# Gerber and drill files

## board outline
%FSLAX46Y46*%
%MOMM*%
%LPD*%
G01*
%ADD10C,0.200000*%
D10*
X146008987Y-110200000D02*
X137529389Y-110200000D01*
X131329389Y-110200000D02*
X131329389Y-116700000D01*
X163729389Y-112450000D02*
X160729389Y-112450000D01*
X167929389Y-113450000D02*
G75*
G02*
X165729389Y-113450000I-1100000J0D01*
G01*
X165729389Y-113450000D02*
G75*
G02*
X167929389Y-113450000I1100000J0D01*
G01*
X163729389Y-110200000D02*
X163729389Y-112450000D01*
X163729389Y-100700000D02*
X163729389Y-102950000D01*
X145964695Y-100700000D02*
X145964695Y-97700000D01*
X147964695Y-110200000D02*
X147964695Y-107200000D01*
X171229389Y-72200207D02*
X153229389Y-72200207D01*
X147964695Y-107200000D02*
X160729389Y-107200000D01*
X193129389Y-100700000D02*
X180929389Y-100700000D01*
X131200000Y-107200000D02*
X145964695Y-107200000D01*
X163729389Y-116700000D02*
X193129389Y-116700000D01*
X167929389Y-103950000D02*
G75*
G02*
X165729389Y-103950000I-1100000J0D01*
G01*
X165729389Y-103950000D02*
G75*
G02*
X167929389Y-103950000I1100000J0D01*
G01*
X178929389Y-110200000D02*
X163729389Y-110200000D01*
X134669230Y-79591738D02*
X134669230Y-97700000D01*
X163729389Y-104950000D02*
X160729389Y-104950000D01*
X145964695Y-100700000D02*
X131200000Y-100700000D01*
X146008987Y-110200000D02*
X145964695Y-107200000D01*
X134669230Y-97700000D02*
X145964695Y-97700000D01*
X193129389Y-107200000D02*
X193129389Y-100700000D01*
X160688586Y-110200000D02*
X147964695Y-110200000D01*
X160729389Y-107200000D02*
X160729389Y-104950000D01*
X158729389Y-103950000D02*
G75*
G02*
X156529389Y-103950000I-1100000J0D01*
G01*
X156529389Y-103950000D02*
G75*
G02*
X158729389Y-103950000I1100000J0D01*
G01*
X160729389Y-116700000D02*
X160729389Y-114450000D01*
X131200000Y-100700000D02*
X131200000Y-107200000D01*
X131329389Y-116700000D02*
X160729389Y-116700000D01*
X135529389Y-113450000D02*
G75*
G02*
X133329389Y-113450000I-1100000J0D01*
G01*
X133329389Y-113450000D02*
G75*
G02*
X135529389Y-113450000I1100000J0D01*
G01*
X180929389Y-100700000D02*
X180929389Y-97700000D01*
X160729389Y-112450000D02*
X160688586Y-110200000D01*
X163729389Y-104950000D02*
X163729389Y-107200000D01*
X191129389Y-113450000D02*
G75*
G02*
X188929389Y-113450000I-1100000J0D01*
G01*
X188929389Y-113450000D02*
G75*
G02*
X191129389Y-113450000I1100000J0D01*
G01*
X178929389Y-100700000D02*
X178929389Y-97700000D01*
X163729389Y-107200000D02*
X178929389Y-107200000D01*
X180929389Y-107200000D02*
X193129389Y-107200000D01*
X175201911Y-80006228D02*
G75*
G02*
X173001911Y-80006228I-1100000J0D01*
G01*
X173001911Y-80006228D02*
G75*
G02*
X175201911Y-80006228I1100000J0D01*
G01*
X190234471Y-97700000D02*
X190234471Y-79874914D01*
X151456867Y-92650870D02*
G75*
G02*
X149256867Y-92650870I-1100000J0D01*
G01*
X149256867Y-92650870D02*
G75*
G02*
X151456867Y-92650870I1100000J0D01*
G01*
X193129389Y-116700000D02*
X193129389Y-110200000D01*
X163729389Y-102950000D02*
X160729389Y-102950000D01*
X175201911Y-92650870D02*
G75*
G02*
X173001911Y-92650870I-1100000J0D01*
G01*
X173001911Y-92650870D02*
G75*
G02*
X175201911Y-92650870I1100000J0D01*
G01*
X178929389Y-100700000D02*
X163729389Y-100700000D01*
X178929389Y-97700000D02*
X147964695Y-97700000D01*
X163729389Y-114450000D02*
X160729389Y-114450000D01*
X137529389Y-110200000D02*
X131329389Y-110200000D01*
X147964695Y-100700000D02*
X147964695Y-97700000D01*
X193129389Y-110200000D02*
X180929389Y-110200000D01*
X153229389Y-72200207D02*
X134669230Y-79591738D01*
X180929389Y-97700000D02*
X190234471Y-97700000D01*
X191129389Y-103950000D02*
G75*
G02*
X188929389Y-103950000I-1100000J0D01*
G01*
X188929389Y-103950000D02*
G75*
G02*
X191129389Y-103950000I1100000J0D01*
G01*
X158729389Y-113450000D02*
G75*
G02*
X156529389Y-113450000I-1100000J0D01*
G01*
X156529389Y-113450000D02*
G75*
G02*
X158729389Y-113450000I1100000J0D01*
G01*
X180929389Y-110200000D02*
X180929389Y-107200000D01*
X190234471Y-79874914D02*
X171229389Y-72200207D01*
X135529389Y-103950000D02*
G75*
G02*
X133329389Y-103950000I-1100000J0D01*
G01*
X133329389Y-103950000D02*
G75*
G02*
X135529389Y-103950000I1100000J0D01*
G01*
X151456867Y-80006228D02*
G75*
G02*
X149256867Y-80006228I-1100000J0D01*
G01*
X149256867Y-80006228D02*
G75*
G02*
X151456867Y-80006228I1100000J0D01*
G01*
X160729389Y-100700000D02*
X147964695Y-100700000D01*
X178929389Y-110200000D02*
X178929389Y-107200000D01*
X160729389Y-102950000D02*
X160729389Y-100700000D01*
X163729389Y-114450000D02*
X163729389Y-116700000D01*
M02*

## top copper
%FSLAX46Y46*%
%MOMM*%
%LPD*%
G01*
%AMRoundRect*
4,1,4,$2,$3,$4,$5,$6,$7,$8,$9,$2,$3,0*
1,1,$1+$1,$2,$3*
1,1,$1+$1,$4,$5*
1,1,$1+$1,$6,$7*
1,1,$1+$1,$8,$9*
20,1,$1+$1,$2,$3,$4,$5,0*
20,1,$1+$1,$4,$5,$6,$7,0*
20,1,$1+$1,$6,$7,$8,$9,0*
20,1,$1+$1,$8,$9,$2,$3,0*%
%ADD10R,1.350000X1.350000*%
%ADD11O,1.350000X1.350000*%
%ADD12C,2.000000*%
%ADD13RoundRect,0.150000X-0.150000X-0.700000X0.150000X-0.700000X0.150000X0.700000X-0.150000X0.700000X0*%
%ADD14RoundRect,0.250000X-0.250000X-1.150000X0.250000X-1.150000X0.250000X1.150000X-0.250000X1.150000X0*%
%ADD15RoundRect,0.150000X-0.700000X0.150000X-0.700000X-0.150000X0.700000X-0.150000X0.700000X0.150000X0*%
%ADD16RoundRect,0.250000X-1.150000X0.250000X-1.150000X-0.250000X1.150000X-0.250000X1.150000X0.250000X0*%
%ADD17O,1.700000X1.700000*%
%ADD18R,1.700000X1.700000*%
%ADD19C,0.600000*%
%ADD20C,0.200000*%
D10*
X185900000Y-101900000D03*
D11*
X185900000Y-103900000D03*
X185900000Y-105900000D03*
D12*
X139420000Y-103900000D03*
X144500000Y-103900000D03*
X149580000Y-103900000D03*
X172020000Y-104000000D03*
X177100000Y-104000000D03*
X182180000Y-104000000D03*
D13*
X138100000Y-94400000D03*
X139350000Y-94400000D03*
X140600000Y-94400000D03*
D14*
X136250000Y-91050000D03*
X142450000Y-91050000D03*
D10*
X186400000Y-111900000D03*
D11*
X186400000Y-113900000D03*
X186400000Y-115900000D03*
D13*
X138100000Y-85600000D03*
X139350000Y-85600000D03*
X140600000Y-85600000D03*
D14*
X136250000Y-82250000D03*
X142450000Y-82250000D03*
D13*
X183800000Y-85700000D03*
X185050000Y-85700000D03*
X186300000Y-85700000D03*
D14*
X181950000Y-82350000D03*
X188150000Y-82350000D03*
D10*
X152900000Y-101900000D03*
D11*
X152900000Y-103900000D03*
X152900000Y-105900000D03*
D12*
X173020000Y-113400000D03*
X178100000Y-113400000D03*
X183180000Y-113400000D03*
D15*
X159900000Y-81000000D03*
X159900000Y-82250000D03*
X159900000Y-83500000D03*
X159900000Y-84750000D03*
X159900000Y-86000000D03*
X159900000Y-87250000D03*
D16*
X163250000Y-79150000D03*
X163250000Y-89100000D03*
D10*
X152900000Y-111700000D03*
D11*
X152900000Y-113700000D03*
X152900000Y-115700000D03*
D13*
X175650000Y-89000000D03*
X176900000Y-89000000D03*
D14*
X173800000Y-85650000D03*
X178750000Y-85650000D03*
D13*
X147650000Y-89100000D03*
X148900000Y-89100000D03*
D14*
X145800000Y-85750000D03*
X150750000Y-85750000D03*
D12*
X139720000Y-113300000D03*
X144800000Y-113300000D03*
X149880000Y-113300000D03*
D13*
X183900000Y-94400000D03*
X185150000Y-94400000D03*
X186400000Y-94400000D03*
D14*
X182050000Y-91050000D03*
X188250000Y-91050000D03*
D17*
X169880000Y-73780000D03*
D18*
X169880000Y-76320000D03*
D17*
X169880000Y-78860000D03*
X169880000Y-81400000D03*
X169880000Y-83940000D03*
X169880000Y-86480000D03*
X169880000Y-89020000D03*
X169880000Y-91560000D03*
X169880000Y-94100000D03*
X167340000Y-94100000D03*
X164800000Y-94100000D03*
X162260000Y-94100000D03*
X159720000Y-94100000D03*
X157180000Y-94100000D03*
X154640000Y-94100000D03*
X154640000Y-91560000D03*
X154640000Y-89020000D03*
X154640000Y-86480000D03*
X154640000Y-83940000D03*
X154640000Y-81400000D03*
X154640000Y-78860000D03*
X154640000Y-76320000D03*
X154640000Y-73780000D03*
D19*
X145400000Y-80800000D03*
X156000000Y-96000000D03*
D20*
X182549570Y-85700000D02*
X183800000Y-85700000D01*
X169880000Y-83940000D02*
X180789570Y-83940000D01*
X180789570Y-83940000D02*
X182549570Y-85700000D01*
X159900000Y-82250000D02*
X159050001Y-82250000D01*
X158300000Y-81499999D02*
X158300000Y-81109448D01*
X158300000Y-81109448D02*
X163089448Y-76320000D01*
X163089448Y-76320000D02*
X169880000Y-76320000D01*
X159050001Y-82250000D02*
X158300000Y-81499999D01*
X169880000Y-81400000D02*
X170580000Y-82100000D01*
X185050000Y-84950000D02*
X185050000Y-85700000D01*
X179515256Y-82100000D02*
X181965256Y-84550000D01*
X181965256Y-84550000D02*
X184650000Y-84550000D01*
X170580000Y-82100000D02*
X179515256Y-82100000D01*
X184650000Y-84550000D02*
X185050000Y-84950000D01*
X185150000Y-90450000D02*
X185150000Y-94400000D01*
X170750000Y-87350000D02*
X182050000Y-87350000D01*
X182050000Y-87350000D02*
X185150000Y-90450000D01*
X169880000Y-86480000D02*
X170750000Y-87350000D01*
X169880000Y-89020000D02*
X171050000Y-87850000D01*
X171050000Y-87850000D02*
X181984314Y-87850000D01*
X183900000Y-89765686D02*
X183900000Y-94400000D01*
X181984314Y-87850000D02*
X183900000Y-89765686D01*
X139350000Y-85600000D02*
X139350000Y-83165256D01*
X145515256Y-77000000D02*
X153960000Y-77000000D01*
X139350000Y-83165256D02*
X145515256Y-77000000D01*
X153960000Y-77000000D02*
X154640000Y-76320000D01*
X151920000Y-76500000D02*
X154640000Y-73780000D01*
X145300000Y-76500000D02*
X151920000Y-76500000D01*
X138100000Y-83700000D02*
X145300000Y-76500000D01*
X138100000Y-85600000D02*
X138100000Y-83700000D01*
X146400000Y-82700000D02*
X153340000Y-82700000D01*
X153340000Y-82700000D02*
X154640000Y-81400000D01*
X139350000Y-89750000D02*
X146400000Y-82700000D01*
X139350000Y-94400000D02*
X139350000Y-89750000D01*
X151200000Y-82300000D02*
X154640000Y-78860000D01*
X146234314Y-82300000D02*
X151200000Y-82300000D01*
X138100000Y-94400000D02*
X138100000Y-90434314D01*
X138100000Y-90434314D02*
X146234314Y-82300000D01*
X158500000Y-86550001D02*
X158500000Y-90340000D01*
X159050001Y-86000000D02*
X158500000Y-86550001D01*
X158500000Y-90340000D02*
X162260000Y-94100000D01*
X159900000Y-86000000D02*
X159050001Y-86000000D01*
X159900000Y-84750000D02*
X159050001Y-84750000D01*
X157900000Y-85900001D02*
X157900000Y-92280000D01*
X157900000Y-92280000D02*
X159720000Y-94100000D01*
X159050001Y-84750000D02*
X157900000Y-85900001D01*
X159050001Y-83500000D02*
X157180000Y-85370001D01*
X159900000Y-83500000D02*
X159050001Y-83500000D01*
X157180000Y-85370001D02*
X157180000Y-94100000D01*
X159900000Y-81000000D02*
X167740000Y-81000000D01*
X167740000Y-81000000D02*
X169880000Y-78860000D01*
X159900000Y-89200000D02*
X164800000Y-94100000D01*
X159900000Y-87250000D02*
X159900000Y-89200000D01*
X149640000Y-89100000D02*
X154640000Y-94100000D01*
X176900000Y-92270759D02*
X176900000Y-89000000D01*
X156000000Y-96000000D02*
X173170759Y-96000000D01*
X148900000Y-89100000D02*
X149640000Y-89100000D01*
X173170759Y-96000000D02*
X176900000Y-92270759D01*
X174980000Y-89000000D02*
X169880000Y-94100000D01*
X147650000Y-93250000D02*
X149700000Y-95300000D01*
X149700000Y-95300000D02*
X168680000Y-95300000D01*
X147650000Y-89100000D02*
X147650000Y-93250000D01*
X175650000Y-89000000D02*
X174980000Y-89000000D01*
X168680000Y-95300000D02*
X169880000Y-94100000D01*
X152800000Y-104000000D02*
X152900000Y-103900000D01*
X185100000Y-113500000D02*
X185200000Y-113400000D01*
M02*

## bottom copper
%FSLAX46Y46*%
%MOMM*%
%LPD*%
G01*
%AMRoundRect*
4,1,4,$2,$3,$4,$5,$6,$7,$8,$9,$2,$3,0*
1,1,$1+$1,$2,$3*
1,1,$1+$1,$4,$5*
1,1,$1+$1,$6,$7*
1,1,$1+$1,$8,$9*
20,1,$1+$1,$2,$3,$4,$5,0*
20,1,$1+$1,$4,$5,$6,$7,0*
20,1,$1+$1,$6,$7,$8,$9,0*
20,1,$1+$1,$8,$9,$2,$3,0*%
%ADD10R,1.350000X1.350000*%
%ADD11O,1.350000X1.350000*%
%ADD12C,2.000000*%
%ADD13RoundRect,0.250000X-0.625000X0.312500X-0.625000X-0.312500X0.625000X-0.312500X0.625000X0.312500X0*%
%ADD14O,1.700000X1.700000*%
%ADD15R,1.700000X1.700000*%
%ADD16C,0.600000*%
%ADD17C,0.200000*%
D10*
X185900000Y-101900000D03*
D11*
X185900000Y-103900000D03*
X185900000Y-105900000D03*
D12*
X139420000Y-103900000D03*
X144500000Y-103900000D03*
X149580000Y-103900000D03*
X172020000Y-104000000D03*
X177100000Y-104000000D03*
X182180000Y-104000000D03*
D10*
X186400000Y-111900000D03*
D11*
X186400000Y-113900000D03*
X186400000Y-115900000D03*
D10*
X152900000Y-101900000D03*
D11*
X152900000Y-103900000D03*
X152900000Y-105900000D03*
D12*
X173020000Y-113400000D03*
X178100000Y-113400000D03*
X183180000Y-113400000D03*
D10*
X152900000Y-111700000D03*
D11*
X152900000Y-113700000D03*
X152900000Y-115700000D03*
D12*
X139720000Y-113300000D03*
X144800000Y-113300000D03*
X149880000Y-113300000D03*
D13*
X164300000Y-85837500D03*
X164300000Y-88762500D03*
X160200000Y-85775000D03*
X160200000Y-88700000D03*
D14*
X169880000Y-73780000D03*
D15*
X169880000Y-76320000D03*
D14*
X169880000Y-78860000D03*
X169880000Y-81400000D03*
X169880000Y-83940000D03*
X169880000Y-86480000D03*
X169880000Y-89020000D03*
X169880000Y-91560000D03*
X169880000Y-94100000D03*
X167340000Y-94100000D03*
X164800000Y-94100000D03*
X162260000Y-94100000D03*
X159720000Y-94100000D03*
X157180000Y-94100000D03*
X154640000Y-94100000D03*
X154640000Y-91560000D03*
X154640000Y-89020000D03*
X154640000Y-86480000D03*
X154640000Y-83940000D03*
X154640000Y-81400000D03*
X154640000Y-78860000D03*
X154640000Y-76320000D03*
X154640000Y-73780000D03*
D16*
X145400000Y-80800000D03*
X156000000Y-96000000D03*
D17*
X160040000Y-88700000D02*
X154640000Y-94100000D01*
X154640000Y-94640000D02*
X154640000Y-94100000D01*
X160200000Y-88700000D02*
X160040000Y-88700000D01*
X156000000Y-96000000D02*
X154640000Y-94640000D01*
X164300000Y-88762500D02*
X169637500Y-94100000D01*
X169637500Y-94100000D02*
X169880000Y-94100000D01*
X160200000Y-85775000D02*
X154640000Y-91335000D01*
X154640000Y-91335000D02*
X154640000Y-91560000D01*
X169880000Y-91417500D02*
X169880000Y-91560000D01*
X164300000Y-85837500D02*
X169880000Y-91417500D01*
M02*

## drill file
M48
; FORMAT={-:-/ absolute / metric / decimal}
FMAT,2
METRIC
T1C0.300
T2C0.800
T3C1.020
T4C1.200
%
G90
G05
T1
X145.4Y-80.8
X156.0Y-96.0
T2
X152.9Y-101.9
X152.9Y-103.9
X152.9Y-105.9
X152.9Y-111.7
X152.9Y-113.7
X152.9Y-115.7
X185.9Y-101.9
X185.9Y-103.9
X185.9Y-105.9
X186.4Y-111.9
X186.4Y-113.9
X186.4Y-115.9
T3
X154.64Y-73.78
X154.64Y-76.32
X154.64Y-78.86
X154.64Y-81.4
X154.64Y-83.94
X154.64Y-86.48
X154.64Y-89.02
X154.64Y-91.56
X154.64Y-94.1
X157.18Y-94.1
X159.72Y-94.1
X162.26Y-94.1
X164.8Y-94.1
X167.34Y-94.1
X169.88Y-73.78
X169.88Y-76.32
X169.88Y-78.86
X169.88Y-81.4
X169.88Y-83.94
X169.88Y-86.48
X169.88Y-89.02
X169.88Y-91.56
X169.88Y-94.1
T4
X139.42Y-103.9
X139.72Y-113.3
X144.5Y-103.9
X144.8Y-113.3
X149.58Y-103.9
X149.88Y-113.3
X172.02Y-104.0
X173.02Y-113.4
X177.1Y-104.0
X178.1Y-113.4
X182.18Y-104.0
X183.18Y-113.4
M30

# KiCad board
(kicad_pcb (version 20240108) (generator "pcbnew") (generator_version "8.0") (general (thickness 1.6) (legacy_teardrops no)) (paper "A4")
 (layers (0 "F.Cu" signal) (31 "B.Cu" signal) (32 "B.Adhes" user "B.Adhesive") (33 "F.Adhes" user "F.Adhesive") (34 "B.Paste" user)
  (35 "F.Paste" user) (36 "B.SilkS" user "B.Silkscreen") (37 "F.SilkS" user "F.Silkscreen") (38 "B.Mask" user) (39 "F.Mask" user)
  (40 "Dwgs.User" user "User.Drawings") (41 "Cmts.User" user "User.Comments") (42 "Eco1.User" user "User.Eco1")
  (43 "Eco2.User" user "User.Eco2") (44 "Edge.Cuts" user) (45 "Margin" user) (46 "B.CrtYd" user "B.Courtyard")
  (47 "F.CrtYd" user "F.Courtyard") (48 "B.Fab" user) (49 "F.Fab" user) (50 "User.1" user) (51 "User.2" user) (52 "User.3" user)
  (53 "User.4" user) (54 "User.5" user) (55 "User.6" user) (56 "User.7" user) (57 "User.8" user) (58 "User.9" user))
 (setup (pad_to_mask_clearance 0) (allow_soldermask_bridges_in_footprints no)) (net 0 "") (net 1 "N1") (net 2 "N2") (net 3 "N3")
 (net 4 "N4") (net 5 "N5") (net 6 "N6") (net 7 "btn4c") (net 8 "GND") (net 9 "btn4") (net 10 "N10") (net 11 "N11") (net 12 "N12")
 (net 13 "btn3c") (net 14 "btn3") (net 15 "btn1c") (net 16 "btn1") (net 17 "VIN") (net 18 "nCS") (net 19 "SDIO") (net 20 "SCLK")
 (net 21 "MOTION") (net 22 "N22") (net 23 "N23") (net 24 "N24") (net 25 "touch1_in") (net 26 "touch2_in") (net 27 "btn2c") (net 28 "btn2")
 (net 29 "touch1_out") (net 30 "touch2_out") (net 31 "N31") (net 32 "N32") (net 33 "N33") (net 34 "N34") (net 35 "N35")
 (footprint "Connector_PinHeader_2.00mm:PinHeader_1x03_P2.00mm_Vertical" (layer "F.Cu") (at 185.9 101.9)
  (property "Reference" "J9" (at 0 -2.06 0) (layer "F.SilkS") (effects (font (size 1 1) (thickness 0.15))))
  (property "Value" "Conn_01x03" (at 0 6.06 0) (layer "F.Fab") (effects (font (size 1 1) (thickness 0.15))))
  (pad "1" thru_hole rect (at 0 0) (size 1.35 1.35) (drill 0.8) (layers "*.Cu" "*.Mask") (remove_unused_layers no) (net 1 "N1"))
  (pad "2" thru_hole oval (at 0 2) (size 1.35 1.35) (drill 0.8) (layers "*.Cu" "*.Mask") (remove_unused_layers no) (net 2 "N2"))
  (pad "3" thru_hole oval (at 0 4) (size 1.35 1.35) (drill 0.8) (layers "*.Cu" "*.Mask") (remove_unused_layers no) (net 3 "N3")))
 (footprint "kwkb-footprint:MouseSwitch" (layer "F.Cu") (at 144.5 103.9 90)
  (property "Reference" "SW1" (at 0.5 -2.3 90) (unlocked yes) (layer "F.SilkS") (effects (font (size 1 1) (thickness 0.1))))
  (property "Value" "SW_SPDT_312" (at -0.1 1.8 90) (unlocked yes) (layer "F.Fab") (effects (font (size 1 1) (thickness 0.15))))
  (pad "1" thru_hole circle (at 0 -5.08 90) (size 2 2) (drill 1.2) (layers "*.Cu" "*.Mask") (remove_unused_layers no) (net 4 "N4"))
  (pad "2" thru_hole circle (at 0 0 90) (size 2 2) (drill 1.2) (layers "*.Cu" "*.Mask") (remove_unused_layers no) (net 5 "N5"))
  (pad "3" thru_hole circle (at 0 5.08 90) (size 2 2) (drill 1.2) (layers "*.Cu" "*.Mask") (remove_unused_layers no) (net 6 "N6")))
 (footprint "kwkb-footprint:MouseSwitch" (layer "F.Cu") (at 177.1 104 90)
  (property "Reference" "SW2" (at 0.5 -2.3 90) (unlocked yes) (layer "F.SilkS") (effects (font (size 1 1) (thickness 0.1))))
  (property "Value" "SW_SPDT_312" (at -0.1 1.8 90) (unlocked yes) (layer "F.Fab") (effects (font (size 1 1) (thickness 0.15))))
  (pad "1" thru_hole circle (at 0 -5.08 90) (size 2 2) (drill 1.2) (layers "*.Cu" "*.Mask") (remove_unused_layers no) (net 1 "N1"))
  (pad "2" thru_hole circle (at 0 0 90) (size 2 2) (drill 1.2) (layers "*.Cu" "*.Mask") (remove_unused_layers no) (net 2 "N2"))
  (pad "3" thru_hole circle (at 0 5.08 90) (size 2 2) (drill 1.2) (layers "*.Cu" "*.Mask") (remove_unused_layers no) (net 3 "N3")))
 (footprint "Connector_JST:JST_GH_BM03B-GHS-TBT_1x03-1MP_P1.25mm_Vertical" (layer "F.Cu") (at 139.35 92.45)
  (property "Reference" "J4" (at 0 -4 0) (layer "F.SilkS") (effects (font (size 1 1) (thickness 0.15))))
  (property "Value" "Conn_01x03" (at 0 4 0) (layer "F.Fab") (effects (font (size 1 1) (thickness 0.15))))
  (pad "1" smd roundrect (at -1.25 1.95) (size 0.6 1.7) (layers "F.Cu" "F.Paste" "F.Mask") (roundrect_rratio 0.25) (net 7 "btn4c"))
  (pad "2" smd roundrect (at 0 1.95) (size 0.6 1.7) (layers "F.Cu" "F.Paste" "F.Mask") (roundrect_rratio 0.25) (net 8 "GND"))
  (pad "3" smd roundrect (at 1.25 1.95) (size 0.6 1.7) (layers "F.Cu" "F.Paste" "F.Mask") (roundrect_rratio 0.25) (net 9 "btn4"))
  (pad "MP" smd roundrect (at -3.1 -1.4) (size 1 2.8) (layers "F.Cu" "F.Paste" "F.Mask") (roundrect_rratio 0.25))
  (pad "MP" smd roundrect (at 3.1 -1.4) (size 1 2.8) (layers "F.Cu" "F.Paste" "F.Mask") (roundrect_rratio 0.25)))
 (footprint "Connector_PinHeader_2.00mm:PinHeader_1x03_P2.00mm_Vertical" (layer "F.Cu") (at 186.4 111.9)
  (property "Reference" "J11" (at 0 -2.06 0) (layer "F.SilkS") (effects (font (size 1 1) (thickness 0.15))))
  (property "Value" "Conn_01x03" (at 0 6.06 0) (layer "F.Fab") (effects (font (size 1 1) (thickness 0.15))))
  (pad "1" thru_hole rect (at 0 0) (size 1.35 1.35) (drill 0.8) (layers "*.Cu" "*.Mask") (remove_unused_layers no) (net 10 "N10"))
  (pad "2" thru_hole oval (at 0 2) (size 1.35 1.35) (drill 0.8) (layers "*.Cu" "*.Mask") (remove_unused_layers no) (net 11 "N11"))
  (pad "3" thru_hole oval (at 0 4) (size 1.35 1.35) (drill 0.8) (layers "*.Cu" "*.Mask") (remove_unused_layers no) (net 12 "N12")))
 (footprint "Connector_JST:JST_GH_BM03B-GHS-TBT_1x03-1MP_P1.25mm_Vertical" (layer "F.Cu") (at 139.35 83.65)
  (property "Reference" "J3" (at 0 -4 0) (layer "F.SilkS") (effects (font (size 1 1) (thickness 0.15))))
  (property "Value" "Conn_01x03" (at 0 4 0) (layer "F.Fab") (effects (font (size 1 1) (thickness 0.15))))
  (pad "1" smd roundrect (at -1.25 1.95) (size 0.6 1.7) (layers "F.Cu" "F.Paste" "F.Mask") (roundrect_rratio 0.25) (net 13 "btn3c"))
  (pad "2" smd roundrect (at 0 1.95) (size 0.6 1.7) (layers "F.Cu" "F.Paste" "F.Mask") (roundrect_rratio 0.25) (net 8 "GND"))
  (pad "3" smd roundrect (at 1.25 1.95) (size 0.6 1.7) (layers "F.Cu" "F.Paste" "F.Mask") (roundrect_rratio 0.25) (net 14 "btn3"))
  (pad "MP" smd roundrect (at -3.1 -1.4) (size 1 2.8) (layers "F.Cu" "F.Paste" "F.Mask") (roundrect_rratio 0.25))
  (pad "MP" smd roundrect (at 3.1 -1.4) (size 1 2.8) (layers "F.Cu" "F.Paste" "F.Mask") (roundrect_rratio 0.25)))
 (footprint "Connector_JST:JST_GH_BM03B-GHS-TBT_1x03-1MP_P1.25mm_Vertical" (layer "F.Cu") (at 185.05 83.75)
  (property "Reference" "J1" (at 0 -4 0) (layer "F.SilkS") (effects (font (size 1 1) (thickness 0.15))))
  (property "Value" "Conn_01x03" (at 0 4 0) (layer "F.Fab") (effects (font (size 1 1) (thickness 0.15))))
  (pad "1" smd roundrect (at -1.25 1.95) (size 0.6 1.7) (layers "F.Cu" "F.Paste" "F.Mask") (roundrect_rratio 0.25) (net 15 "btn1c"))
  (pad "2" smd roundrect (at 0 1.95) (size 0.6 1.7) (layers "F.Cu" "F.Paste" "F.Mask") (roundrect_rratio 0.25) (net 8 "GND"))
  (pad "3" smd roundrect (at 1.25 1.95) (size 0.6 1.7) (layers "F.Cu" "F.Paste" "F.Mask") (roundrect_rratio 0.25) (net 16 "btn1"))
  (pad "MP" smd roundrect (at -3.1 -1.4) (size 1 2.8) (layers "F.Cu" "F.Paste" "F.Mask") (roundrect_rratio 0.25))
  (pad "MP" smd roundrect (at 3.1 -1.4) (size 1 2.8) (layers "F.Cu" "F.Paste" "F.Mask") (roundrect_rratio 0.25)))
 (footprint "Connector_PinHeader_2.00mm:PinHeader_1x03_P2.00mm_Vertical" (layer "F.Cu") (at 152.9 101.9)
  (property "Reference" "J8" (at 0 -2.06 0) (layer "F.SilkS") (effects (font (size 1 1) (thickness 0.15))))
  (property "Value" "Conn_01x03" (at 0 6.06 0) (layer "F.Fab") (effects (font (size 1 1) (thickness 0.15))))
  (pad "1" thru_hole rect (at 0 0) (size 1.35 1.35) (drill 0.8) (layers "*.Cu" "*.Mask") (remove_unused_layers no) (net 4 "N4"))
  (pad "2" thru_hole oval (at 0 2) (size 1.35 1.35) (drill 0.8) (layers "*.Cu" "*.Mask") (remove_unused_layers no) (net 5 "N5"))
  (pad "3" thru_hole oval (at 0 4) (size 1.35 1.35) (drill 0.8) (layers "*.Cu" "*.Mask") (remove_unused_layers no) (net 6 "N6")))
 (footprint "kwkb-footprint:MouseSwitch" (layer "F.Cu") (at 178.1 113.4 90)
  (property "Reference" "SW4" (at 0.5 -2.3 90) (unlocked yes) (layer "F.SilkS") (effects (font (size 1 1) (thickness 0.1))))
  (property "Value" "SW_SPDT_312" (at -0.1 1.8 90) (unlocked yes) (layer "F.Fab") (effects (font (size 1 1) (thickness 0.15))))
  (pad "1" thru_hole circle (at 0 -5.08 90) (size 2 2) (drill 1.2) (layers "*.Cu" "*.Mask") (remove_unused_layers no) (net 10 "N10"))
  (pad "2" thru_hole circle (at 0 0 90) (size 2 2) (drill 1.2) (layers "*.Cu" "*.Mask") (remove_unused_layers no) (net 11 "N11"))
  (pad "3" thru_hole circle (at 0 5.08 90) (size 2 2) (drill 1.2) (layers "*.Cu" "*.Mask") (remove_unused_layers no) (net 12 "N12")))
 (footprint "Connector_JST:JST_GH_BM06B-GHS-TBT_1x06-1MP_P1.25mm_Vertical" (layer "F.Cu") (at 161.85 84.125 -90)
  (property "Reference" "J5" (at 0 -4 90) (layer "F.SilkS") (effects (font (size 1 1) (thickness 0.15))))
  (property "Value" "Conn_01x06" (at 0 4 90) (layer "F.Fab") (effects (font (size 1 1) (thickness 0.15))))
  (pad "1" smd roundrect (at -3.125 1.95 270) (size 0.6 1.7) (layers "F.Cu" "F.Paste" "F.Mask") (roundrect_rratio 0.25) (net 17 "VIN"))
  (pad "2" smd roundrect (at -1.875 1.95 270) (size 0.6 1.7) (layers "F.Cu" "F.Paste" "F.Mask") (roundrect_rratio 0.25) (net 8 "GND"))
  (pad "3" smd roundrect (at -0.625 1.95 270) (size 0.6 1.7) (layers "F.Cu" "F.Paste" "F.Mask") (roundrect_rratio 0.25) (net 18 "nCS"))
  (pad "4" smd roundrect (at 0.625 1.95 270) (size 0.6 1.7) (layers "F.Cu" "F.Paste" "F.Mask") (roundrect_rratio 0.25) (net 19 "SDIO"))
  (pad "5" smd roundrect (at 1.875 1.95 270) (size 0.6 1.7) (layers "F.Cu" "F.Paste" "F.Mask") (roundrect_rratio 0.25) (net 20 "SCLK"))
  (pad "6" smd roundrect (at 3.125 1.95 270) (size 0.6 1.7) (layers "F.Cu" "F.Paste" "F.Mask") (roundrect_rratio 0.25) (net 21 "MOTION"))
  (pad "MP" smd roundrect (at -4.975 -1.4 270) (size 1 2.8) (layers "F.Cu" "F.Paste" "F.Mask") (roundrect_rratio 0.25))
  (pad "MP" smd roundrect (at 4.975 -1.4 270) (size 1 2.8) (layers "F.Cu" "F.Paste" "F.Mask") (roundrect_rratio 0.25)))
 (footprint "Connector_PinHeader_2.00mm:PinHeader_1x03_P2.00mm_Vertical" (layer "F.Cu") (at 152.9 111.7)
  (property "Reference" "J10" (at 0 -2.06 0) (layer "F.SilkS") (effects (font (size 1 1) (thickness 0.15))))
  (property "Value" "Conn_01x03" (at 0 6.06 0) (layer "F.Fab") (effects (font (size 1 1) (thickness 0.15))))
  (pad "1" thru_hole rect (at 0 0) (size 1.35 1.35) (drill 0.8) (layers "*.Cu" "*.Mask") (remove_unused_layers no) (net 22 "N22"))
  (pad "2" thru_hole oval (at 0 2) (size 1.35 1.35) (drill 0.8) (layers "*.Cu" "*.Mask") (remove_unused_layers no) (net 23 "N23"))
  (pad "3" thru_hole oval (at 0 4) (size 1.35 1.35) (drill 0.8) (layers "*.Cu" "*.Mask") (remove_unused_layers no) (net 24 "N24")))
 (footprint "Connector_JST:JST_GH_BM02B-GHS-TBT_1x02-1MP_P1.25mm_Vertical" (layer "F.Cu") (at 176.275 87.05)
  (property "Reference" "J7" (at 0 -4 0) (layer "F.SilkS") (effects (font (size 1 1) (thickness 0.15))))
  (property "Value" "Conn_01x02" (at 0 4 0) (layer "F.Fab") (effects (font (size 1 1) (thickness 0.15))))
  (pad "1" smd roundrect (at -0.625 1.95) (size 0.6 1.7) (layers "F.Cu" "F.Paste" "F.Mask") (roundrect_rratio 0.25) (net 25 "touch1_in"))
  (pad "2" smd roundrect (at 0.625 1.95) (size 0.6 1.7) (layers "F.Cu" "F.Paste" "F.Mask") (roundrect_rratio 0.25) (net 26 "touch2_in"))
  (pad "MP" smd roundrect (at -2.475 -1.4) (size 1 2.8) (layers "F.Cu" "F.Paste" "F.Mask") (roundrect_rratio 0.25))
  (pad "MP" smd roundrect (at 2.475 -1.4) (size 1 2.8) (layers "F.Cu" "F.Paste" "F.Mask") (roundrect_rratio 0.25)))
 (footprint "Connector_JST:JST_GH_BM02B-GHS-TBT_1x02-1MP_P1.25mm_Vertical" (layer "F.Cu") (at 148.275 87.15)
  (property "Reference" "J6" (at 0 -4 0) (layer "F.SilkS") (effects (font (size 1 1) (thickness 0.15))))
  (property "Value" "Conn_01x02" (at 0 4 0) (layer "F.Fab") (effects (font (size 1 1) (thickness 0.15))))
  (pad "1" smd roundrect (at -0.625 1.95) (size 0.6 1.7) (layers "F.Cu" "F.Paste" "F.Mask") (roundrect_rratio 0.25) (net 25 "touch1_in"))
  (pad "2" smd roundrect (at 0.625 1.95) (size 0.6 1.7) (layers "F.Cu" "F.Paste" "F.Mask") (roundrect_rratio 0.25) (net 26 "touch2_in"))
  (pad "MP" smd roundrect (at -2.475 -1.4) (size 1 2.8) (layers "F.Cu" "F.Paste" "F.Mask") (roundrect_rratio 0.25))
  (pad "MP" smd roundrect (at 2.475 -1.4) (size 1 2.8) (layers "F.Cu" "F.Paste" "F.Mask") (roundrect_rratio 0.25)))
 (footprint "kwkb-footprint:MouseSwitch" (layer "F.Cu") (at 144.8 113.3 90)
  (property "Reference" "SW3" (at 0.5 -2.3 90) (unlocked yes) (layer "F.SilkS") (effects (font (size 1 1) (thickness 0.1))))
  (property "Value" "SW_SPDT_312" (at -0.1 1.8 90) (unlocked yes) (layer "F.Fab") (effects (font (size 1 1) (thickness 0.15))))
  (pad "1" thru_hole circle (at 0 -5.08 90) (size 2 2) (drill 1.2) (layers "*.Cu" "*.Mask") (remove_unused_layers no) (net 22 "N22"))
  (pad "2" thru_hole circle (at 0 0 90) (size 2 2) (drill 1.2) (layers "*.Cu" "*.Mask") (remove_unused_layers no) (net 23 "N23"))
  (pad "3" thru_hole circle (at 0 5.08 90) (size 2 2) (drill 1.2) (layers "*.Cu" "*.Mask") (remove_unused_layers no) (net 24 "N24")))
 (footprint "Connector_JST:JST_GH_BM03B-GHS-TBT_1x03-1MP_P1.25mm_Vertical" (layer "F.Cu") (at 185.15 92.45)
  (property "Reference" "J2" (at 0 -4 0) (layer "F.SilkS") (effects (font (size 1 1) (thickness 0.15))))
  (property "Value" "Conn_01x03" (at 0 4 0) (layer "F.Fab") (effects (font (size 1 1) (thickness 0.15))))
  (pad "1" smd roundrect (at -1.25 1.95) (size 0.6 1.7) (layers "F.Cu" "F.Paste" "F.Mask") (roundrect_rratio 0.25) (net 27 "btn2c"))
  (pad "2" smd roundrect (at 0 1.95) (size 0.6 1.7) (layers "F.Cu" "F.Paste" "F.Mask") (roundrect_rratio 0.25) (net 8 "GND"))
  (pad "3" smd roundrect (at 1.25 1.95) (size 0.6 1.7) (layers "F.Cu" "F.Paste" "F.Mask") (roundrect_rratio 0.25) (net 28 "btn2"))
  (pad "MP" smd roundrect (at -3.1 -1.4) (size 1 2.8) (layers "F.Cu" "F.Paste" "F.Mask") (roundrect_rratio 0.25))
  (pad "MP" smd roundrect (at 3.1 -1.4) (size 1 2.8) (layers "F.Cu" "F.Paste" "F.Mask") (roundrect_rratio 0.25)))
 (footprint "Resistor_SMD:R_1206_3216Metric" (layer "B.Cu") (at 164.3 87.3 -90)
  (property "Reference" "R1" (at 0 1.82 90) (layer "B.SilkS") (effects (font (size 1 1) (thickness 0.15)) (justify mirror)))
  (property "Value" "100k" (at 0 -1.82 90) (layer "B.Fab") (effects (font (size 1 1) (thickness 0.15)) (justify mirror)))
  (pad "1" smd roundrect (at -1.4625 0 270) (size 1.125 1.75) (layers "B.Cu" "B.Paste" "B.Mask") (roundrect_rratio 0.222222)
   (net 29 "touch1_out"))
  (pad "2" smd roundrect (at 1.4625 0 270) (size 1.125 1.75) (layers "B.Cu" "B.Paste" "B.Mask") (roundrect_rratio 0.222222)
   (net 25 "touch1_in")))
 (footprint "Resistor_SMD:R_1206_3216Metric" (layer "B.Cu") (at 160.2 87.2375 -90)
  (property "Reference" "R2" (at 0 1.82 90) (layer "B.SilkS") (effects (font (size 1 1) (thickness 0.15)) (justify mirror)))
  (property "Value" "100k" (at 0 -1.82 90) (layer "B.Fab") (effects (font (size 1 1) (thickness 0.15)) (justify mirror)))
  (pad "1" smd roundrect (at -1.4625 0 270) (size 1.125 1.75) (layers "B.Cu" "B.Paste" "B.Mask") (roundrect_rratio 0.222222)
   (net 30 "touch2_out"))
  (pad "2" smd roundrect (at 1.4625 0 270) (size 1.125 1.75) (layers "B.Cu" "B.Paste" "B.Mask") (roundrect_rratio 0.222222)
   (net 26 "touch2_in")))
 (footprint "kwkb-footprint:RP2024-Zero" (layer "B.Cu") (at 162.26 72.19 180)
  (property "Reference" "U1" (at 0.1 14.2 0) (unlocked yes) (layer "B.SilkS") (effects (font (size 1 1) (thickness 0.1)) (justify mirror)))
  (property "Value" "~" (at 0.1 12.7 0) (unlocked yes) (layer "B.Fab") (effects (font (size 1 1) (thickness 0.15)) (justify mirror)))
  (pad "1" thru_hole oval (at -7.62 -1.59 180) (size 1.7 1.7) (drill 1.02) (layers "*.Cu" "*.Mask") (remove_unused_layers no) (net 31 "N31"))
  (pad "2" thru_hole rect (at -7.62 -4.13 180) (size 1.7 1.7) (drill 1.02) (layers "*.Cu" "*.Mask") (remove_unused_layers no) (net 8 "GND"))
  (pad "3" thru_hole oval (at -7.62 -6.67 180) (size 1.7 1.7) (drill 1.02) (layers "*.Cu" "*.Mask") (remove_unused_layers no) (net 17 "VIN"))
  (pad "4" thru_hole oval (at -7.62 -9.21 180) (size 1.7 1.7) (drill 1.02) (layers "*.Cu" "*.Mask") (remove_unused_layers no)
   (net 16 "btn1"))
  (pad "5" thru_hole oval (at -7.62 -11.75 180) (size 1.7 1.7) (drill 1.02) (layers "*.Cu" "*.Mask") (remove_unused_layers no)
   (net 15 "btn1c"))
  (pad "6" thru_hole oval (at -7.62 -14.29 180) (size 1.7 1.7) (drill 1.02) (layers "*.Cu" "*.Mask") (remove_unused_layers no)
   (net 28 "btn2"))
  (pad "7" thru_hole oval (at -7.62 -16.83 180) (size 1.7 1.7) (drill 1.02) (layers "*.Cu" "*.Mask") (remove_unused_layers no)
   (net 27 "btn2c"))
  (pad "8" thru_hole oval (at -7.62 -19.37 180) (size 1.7 1.7) (drill 1.02) (layers "*.Cu" "*.Mask") (remove_unused_layers no)
   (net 29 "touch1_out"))
  (pad "9" thru_hole oval (at -7.62 -21.91 180) (size 1.7 1.7) (drill 1.02) (layers "*.Cu" "*.Mask") (remove_unused_layers no)
   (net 25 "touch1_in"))
  (pad "10" thru_hole oval (at -5.08 -21.91 180) (size 1.7 1.7) (drill 1.02) (layers "*.Cu" "*.Mask") (remove_unused_layers no)
   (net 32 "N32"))
  (pad "11" thru_hole oval (at -2.54 -21.91 180) (size 1.7 1.7) (drill 1.02) (layers "*.Cu" "*.Mask") (remove_unused_layers no)
   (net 21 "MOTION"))
  (pad "12" thru_hole oval (at 0 -21.91 180) (size 1.7 1.7) (drill 1.02) (layers "*.Cu" "*.Mask") (remove_unused_layers no) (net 20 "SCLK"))
  (pad "13" thru_hole oval (at 2.54 -21.91 180) (size 1.7 1.7) (drill 1.02) (layers "*.Cu" "*.Mask") (remove_unused_layers no)
   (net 19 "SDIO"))
  (pad "14" thru_hole oval (at 5.08 -21.91 180) (size 1.7 1.7) (drill 1.02) (layers "*.Cu" "*.Mask") (remove_unused_layers no)
   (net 18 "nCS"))
  (pad "15" thru_hole oval (at 7.62 -21.91 180) (size 1.7 1.7) (drill 1.02) (layers "*.Cu" "*.Mask") (remove_unused_layers no)
   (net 26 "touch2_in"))
  (pad "16" thru_hole oval (at 7.62 -19.37 180) (size 1.7 1.7) (drill 1.02) (layers "*.Cu" "*.Mask") (remove_unused_layers no)
   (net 30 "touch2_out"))
  (pad "17" thru_hole oval (at 7.62 -16.83 180) (size 1.7 1.7) (drill 1.02) (layers "*.Cu" "*.Mask") (remove_unused_layers no)
   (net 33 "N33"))
  (pad "18" thru_hole oval (at 7.62 -14.29 180) (size 1.7 1.7) (drill 1.02) (layers "*.Cu" "*.Mask") (remove_unused_layers no)
   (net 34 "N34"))
  (pad "19" thru_hole oval (at 7.62 -11.75 180) (size 1.7 1.7) (drill 1.02) (layers "*.Cu" "*.Mask") (remove_unused_layers no)
   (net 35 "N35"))
  (pad "20" thru_hole oval (at 7.62 -9.21 180) (size 1.7 1.7) (drill 1.02) (layers "*.Cu" "*.Mask") (remove_unused_layers no) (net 9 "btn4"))
  (pad "21" thru_hole oval (at 7.62 -6.67 180) (size 1.7 1.7) (drill 1.02) (layers "*.Cu" "*.Mask") (remove_unused_layers no)
   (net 7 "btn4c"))
  (pad "22" thru_hole oval (at 7.62 -4.13 180) (size 1.7 1.7) (drill 1.02) (layers "*.Cu" "*.Mask") (remove_unused_layers no)
   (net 14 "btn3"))
  (pad "23" thru_hole oval (at 7.62 -1.59 180) (size 1.7 1.7) (drill 1.02) (layers "*.Cu" "*.Mask") (remove_unused_layers no)
   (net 13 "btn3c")))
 (gr_line (start 146.008987 110.2) (end 137.529389 110.2) (stroke (width 0.2) (type default)) (layer "Edge.Cuts"))
 (gr_line (start 131.329389 110.2) (end 131.329389 116.7) (stroke (width 0.2) (type default)) (layer "Edge.Cuts"))
 (gr_line (start 163.729389 112.45) (end 160.729389 112.45) (stroke (width 0.2) (type default)) (layer "Edge.Cuts"))
 (gr_circle (center 166.829389 113.45) (end 165.729389 113.45) (stroke (width 0.2) (type default)) (fill none) (layer "Edge.Cuts"))
 (gr_line (start 163.729389 110.2) (end 163.729389 112.45) (stroke (width 0.2) (type default)) (layer "Edge.Cuts"))
 (gr_line (start 163.729389 100.7) (end 163.729389 102.95) (stroke (width 0.2) (type default)) (layer "Edge.Cuts"))
 (gr_line (start 145.964695 100.7) (end 145.964695 97.7) (stroke (width 0.2) (type default)) (layer "Edge.Cuts"))
 (gr_line (start 147.964695 110.2) (end 147.964695 107.2) (stroke (width 0.2) (type default)) (layer "Edge.Cuts"))
 (gr_line (start 171.229389 72.200207) (end 153.229389 72.200207) (stroke (width 0.2) (type default)) (layer "Edge.Cuts"))
 (gr_line (start 147.964695 107.2) (end 160.729389 107.2) (stroke (width 0.2) (type default)) (layer "Edge.Cuts"))
 (gr_line (start 193.129389 100.7) (end 180.929389 100.7) (stroke (width 0.2) (type default)) (layer "Edge.Cuts"))
 (gr_line (start 131.2 107.2) (end 145.964695 107.2) (stroke (width 0.2) (type default)) (layer "Edge.Cuts"))
 (gr_line (start 163.729389 116.7) (end 193.129389 116.7) (stroke (width 0.2) (type default)) (layer "Edge.Cuts"))
 (gr_circle (center 166.829389 103.95) (end 165.729389 103.95) (stroke (width 0.2) (type default)) (fill none) (layer "Edge.Cuts"))
 (gr_line (start 178.929389 110.2) (end 163.729389 110.2) (stroke (width 0.2) (type default)) (layer "Edge.Cuts"))
 (gr_line (start 134.66923 79.591738) (end 134.66923 97.7) (stroke (width 0.2) (type default)) (layer "Edge.Cuts"))
 (gr_line (start 163.729389 104.95) (end 160.729389 104.95) (stroke (width 0.2) (type default)) (layer "Edge.Cuts"))
 (gr_line (start 145.964695 100.7) (end 131.2 100.7) (stroke (width 0.2) (type default)) (layer "Edge.Cuts"))
 (gr_line (start 146.008987 110.2) (end 145.964695 107.2) (stroke (width 0.2) (type default)) (layer "Edge.Cuts"))
 (gr_line (start 134.66923 97.7) (end 145.964695 97.7) (stroke (width 0.2) (type default)) (layer "Edge.Cuts"))
 (gr_line (start 193.129389 107.2) (end 193.129389 100.7) (stroke (width 0.2) (type default)) (layer "Edge.Cuts"))
 (gr_line (start 160.688586 110.2) (end 147.964695 110.2) (stroke (width 0.2) (type default)) (layer "Edge.Cuts"))
 (gr_line (start 160.729389 107.2) (end 160.729389 104.95) (stroke (width 0.2) (type default)) (layer "Edge.Cuts"))
 (gr_circle (center 157.629389 103.95) (end 156.529389 103.95) (stroke (width 0.2) (type default)) (fill none) (layer "Edge.Cuts"))
 (gr_line (start 160.729389 116.7) (end 160.729389 114.45) (stroke (width 0.2) (type default)) (layer "Edge.Cuts"))
 (gr_line (start 131.2 100.7) (end 131.2 107.2) (stroke (width 0.2) (type default)) (layer "Edge.Cuts"))
 (gr_line (start 131.329389 116.7) (end 160.729389 116.7) (stroke (width 0.2) (type default)) (layer "Edge.Cuts"))
 (gr_circle (center 134.429389 113.45) (end 133.329389 113.45) (stroke (width 0.2) (type default)) (fill none) (layer "Edge.Cuts"))
 (gr_line (start 180.929389 100.7) (end 180.929389 97.7) (stroke (width 0.2) (type default)) (layer "Edge.Cuts"))
 (gr_line (start 160.729389 112.45) (end 160.688586 110.2) (stroke (width 0.2) (type default)) (layer "Edge.Cuts"))
 (gr_line (start 163.729389 104.95) (end 163.729389 107.2) (stroke (width 0.2) (type default)) (layer "Edge.Cuts"))
 (gr_circle (center 190.029389 113.45) (end 188.929389 113.45) (stroke (width 0.2) (type default)) (fill none) (layer "Edge.Cuts"))
 (gr_line (start 178.929389 100.7) (end 178.929389 97.7) (stroke (width 0.2) (type default)) (layer "Edge.Cuts"))
 (gr_line (start 163.729389 107.2) (end 178.929389 107.2) (stroke (width 0.2) (type default)) (layer "Edge.Cuts"))
 (gr_line (start 180.929389 107.2) (end 193.129389 107.2) (stroke (width 0.2) (type default)) (layer "Edge.Cuts"))
 (gr_circle (center 174.101911 80.006228) (end 173.001911 80.006228) (stroke (width 0.2) (type default)) (fill none) (layer "Edge.Cuts"))
 (gr_line (start 190.234471 97.7) (end 190.234471 79.874914) (stroke (width 0.2) (type default)) (layer "Edge.Cuts"))
 (gr_circle (center 150.356867 92.65087) (end 149.256867 92.65087) (stroke (width 0.2) (type default)) (fill none) (layer "Edge.Cuts"))
 (gr_line (start 193.129389 116.7) (end 193.129389 110.2) (stroke (width 0.2) (type default)) (layer "Edge.Cuts"))
 (gr_line (start 163.729389 102.95) (end 160.729389 102.95) (stroke (width 0.2) (type default)) (layer "Edge.Cuts"))
 (gr_circle (center 174.101911 92.65087) (end 173.001911 92.65087) (stroke (width 0.2) (type default)) (fill none) (layer "Edge.Cuts"))
 (gr_line (start 178.929389 100.7) (end 163.729389 100.7) (stroke (width 0.2) (type default)) (layer "Edge.Cuts"))
 (gr_line (start 178.929389 97.7) (end 147.964695 97.7) (stroke (width 0.2) (type default)) (layer "Edge.Cuts"))
 (gr_line (start 163.729389 114.45) (end 160.729389 114.45) (stroke (width 0.2) (type default)) (layer "Edge.Cuts"))
 (gr_line (start 137.529389 110.2) (end 131.329389 110.2) (stroke (width 0.2) (type default)) (layer "Edge.Cuts"))
 (gr_line (start 147.964695 100.7) (end 147.964695 97.7) (stroke (width 0.2) (type default)) (layer "Edge.Cuts"))
 (gr_line (start 193.129389 110.2) (end 180.929389 110.2) (stroke (width 0.2) (type default)) (layer "Edge.Cuts"))
 (gr_line (start 153.229389 72.200207) (end 134.66923 79.591738) (stroke (width 0.2) (type default)) (layer "Edge.Cuts"))
 (gr_line (start 180.929389 97.7) (end 190.234471 97.7) (stroke (width 0.2) (type default)) (layer "Edge.Cuts"))
 (gr_circle (center 190.029389 103.95) (end 188.929389 103.95) (stroke (width 0.2) (type default)) (fill none) (layer "Edge.Cuts"))
 (gr_circle (center 157.629389 113.45) (end 156.529389 113.45) (stroke (width 0.2) (type default)) (fill none) (layer "Edge.Cuts"))
 (gr_line (start 180.929389 110.2) (end 180.929389 107.2) (stroke (width 0.2) (type default)) (layer "Edge.Cuts"))
 (gr_line (start 190.234471 79.874914) (end 171.229389 72.200207) (stroke (width 0.2) (type default)) (layer "Edge.Cuts"))
 (gr_circle (center 134.429389 103.95) (end 133.329389 103.95) (stroke (width 0.2) (type default)) (fill none) (layer "Edge.Cuts"))
 (gr_circle (center 150.356867 80.006228) (end 149.256867 80.006228) (stroke (width 0.2) (type default)) (fill none) (layer "Edge.Cuts"))
 (gr_line (start 160.729389 100.7) (end 147.964695 100.7) (stroke (width 0.2) (type default)) (layer "Edge.Cuts"))
 (gr_line (start 178.929389 110.2) (end 178.929389 107.2) (stroke (width 0.2) (type default)) (layer "Edge.Cuts"))
 (gr_line (start 160.729389 102.95) (end 160.729389 100.7) (stroke (width 0.2) (type default)) (layer "Edge.Cuts"))
 (gr_line (start 163.729389 114.45) (end 163.729389 116.7) (stroke (width 0.2) (type default)) (layer "Edge.Cuts"))
 (segment (start 182.54957 85.7) (end 183.8 85.7) (width 0.2) (layer "F.Cu") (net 15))
 (segment (start 169.88 83.94) (end 180.78957 83.94) (width 0.2) (layer "F.Cu") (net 15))
 (segment (start 180.78957 83.94) (end 182.54957 85.7) (width 0.2) (layer "F.Cu") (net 15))
 (segment (start 159.9 82.25) (end 159.050001 82.25) (width 0.2) (layer "F.Cu") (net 8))
 (segment (start 158.3 81.499999) (end 158.3 81.109448) (width 0.2) (layer "F.Cu") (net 8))
 (segment (start 158.3 81.109448) (end 163.089448 76.32) (width 0.2) (layer "F.Cu") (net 8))
 (segment (start 163.089448 76.32) (end 169.88 76.32) (width 0.2) (layer "F.Cu") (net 8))
 (segment (start 159.050001 82.25) (end 158.3 81.499999) (width 0.2) (layer "F.Cu") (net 8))
 (via (at 145.4 80.8) (size 0.6) (drill 0.3) (layers "F.Cu" "B.Cu") (free yes) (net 8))
 (segment (start 169.88 81.4) (end 170.58 82.1) (width 0.2) (layer "F.Cu") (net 16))
 (segment (start 185.05 84.95) (end 185.05 85.7) (width 0.2) (layer "F.Cu") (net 16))
 (segment (start 179.515256 82.1) (end 181.965256 84.55) (width 0.2) (layer "F.Cu") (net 16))
 (segment (start 181.965256 84.55) (end 184.65 84.55) (width 0.2) (layer "F.Cu") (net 16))
 (segment (start 170.58 82.1) (end 179.515256 82.1) (width 0.2) (layer "F.Cu") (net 16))
 (segment (start 184.65 84.55) (end 185.05 84.95) (width 0.2) (layer "F.Cu") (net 16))
 (segment (start 185.15 90.45) (end 185.15 94.4) (width 0.2) (layer "F.Cu") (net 28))
 (segment (start 170.75 87.35) (end 182.05 87.35) (width 0.2) (layer "F.Cu") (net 28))
 (segment (start 182.05 87.35) (end 185.15 90.45) (width 0.2) (layer "F.Cu") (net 28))
 (segment (start 169.88 86.48) (end 170.75 87.35) (width 0.2) (layer "F.Cu") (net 28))
 (segment (start 169.88 89.02) (end 171.05 87.85) (width 0.2) (layer "F.Cu") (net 27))
 (segment (start 171.05 87.85) (end 181.984314 87.85) (width 0.2) (layer "F.Cu") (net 27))
 (segment (start 183.9 89.765686) (end 183.9 94.4) (width 0.2) (layer "F.Cu") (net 27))
 (segment (start 181.984314 87.85) (end 183.9 89.765686) (width 0.2) (layer "F.Cu") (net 27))
 (segment (start 139.35 85.6) (end 139.35 83.165256) (width 0.2) (layer "F.Cu") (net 14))
 (segment (start 145.515256 77) (end 153.96 77) (width 0.2) (layer "F.Cu") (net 14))
 (segment (start 139.35 83.165256) (end 145.515256 77) (width 0.2) (layer "F.Cu") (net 14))
 (segment (start 153.96 77) (end 154.64 76.32) (width 0.2) (layer "F.Cu") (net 14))
 (segment (start 151.92 76.5) (end 154.64 73.78) (width 0.2) (layer "F.Cu") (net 13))
 (segment (start 145.3 76.5) (end 151.92 76.5) (width 0.2) (layer "F.Cu") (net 13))
 (segment (start 138.1 83.7) (end 145.3 76.5) (width 0.2) (layer "F.Cu") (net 13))
 (segment (start 138.1 85.6) (end 138.1 83.7) (width 0.2) (layer "F.Cu") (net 13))
 (segment (start 146.4 82.7) (end 153.34 82.7) (width 0.2) (layer "F.Cu") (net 9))
 (segment (start 153.34 82.7) (end 154.64 81.4) (width 0.2) (layer "F.Cu") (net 9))
 (segment (start 139.35 89.75) (end 146.4 82.7) (width 0.2) (layer "F.Cu") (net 9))
 (segment (start 139.35 94.4) (end 139.35 89.75) (width 0.2) (layer "F.Cu") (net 9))
 (segment (start 151.2 82.3) (end 154.64 78.86) (width 0.2) (layer "F.Cu") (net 7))
 (segment (start 146.234314 82.3) (end 151.2 82.3) (width 0.2) (layer "F.Cu") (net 7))
 (segment (start 138.1 94.4) (end 138.1 90.434314) (width 0.2) (layer "F.Cu") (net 7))
 (segment (start 138.1 90.434314) (end 146.234314 82.3) (width 0.2) (layer "F.Cu") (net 7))
 (segment (start 158.5 86.550001) (end 158.5 90.34) (width 0.2) (layer "F.Cu") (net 20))
 (segment (start 159.050001 86) (end 158.5 86.550001) (width 0.2) (layer "F.Cu") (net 20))
 (segment (start 158.5 90.34) (end 162.26 94.1) (width 0.2) (layer "F.Cu") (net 20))
 (segment (start 159.9 86) (end 159.050001 86) (width 0.2) (layer "F.Cu") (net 20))
 (segment (start 159.9 84.75) (end 159.050001 84.75) (width 0.2) (layer "F.Cu") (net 19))
 (segment (start 157.9 85.900001) (end 157.9 92.28) (width 0.2) (layer "F.Cu") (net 19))
 (segment (start 157.9 92.28) (end 159.72 94.1) (width 0.2) (layer "F.Cu") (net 19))
 (segment (start 159.050001 84.75) (end 157.9 85.900001) (width 0.2) (layer "F.Cu") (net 19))
 (segment (start 159.050001 83.5) (end 157.18 85.370001) (width 0.2) (layer "F.Cu") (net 18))
 (segment (start 159.9 83.5) (end 159.050001 83.5) (width 0.2) (layer "F.Cu") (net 18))
 (segment (start 157.18 85.370001) (end 157.18 94.1) (width 0.2) (layer "F.Cu") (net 18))
 (segment (start 159.9 81) (end 167.74 81) (width 0.2) (layer "F.Cu") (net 17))
 (segment (start 167.74 81) (end 169.88 78.86) (width 0.2) (layer "F.Cu") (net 17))
 (segment (start 159.9 89.2) (end 164.8 94.1) (width 0.2) (layer "F.Cu") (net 21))
 (segment (start 159.9 87.25) (end 159.9 89.2) (width 0.2) (layer "F.Cu") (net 21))
 (segment (start 149.64 89.1) (end 154.64 94.1) (width 0.2) (layer "F.Cu") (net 26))
 (segment (start 176.9 92.270759) (end 176.9 89) (width 0.2) (layer "F.Cu") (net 26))
 (segment (start 156 96) (end 173.170759 96) (width 0.2) (layer "F.Cu") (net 26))
 (segment (start 148.9 89.1) (end 149.64 89.1) (width 0.2) (layer "F.Cu") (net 26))
 (segment (start 173.170759 96) (end 176.9 92.270759) (width 0.2) (layer "F.Cu") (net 26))
 (via (at 156 96) (size 0.6) (drill 0.3) (layers "F.Cu" "B.Cu") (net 26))
 (segment (start 160.04 88.7) (end 154.64 94.1) (width 0.2) (layer "B.Cu") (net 26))
 (segment (start 154.64 94.64) (end 154.64 94.1) (width 0.2) (layer "B.Cu") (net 26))
 (segment (start 160.2 88.7) (end 160.04 88.7) (width 0.2) (layer "B.Cu") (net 26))
 (segment (start 156 96) (end 154.64 94.64) (width 0.2) (layer "B.Cu") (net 26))
 (segment (start 174.98 89) (end 169.88 94.1) (width 0.2) (layer "F.Cu") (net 25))
 (segment (start 147.65 93.25) (end 149.7 95.3) (width 0.2) (layer "F.Cu") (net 25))
 (segment (start 149.7 95.3) (end 168.68 95.3) (width 0.2) (layer "F.Cu") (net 25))
 (segment (start 147.65 89.1) (end 147.65 93.25) (width 0.2) (layer "F.Cu") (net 25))
 (segment (start 175.65 89) (end 174.98 89) (width 0.2) (layer "F.Cu") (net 25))
 (segment (start 168.68 95.3) (end 169.88 94.1) (width 0.2) (layer "F.Cu") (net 25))
 (segment (start 164.3 88.7625) (end 169.6375 94.1) (width 0.2) (layer "B.Cu") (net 25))
 (segment (start 169.6375 94.1) (end 169.88 94.1) (width 0.2) (layer "B.Cu") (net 25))
 (segment (start 160.2 85.775) (end 154.64 91.335) (width 0.2) (layer "B.Cu") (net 30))
 (segment (start 154.64 91.335) (end 154.64 91.56) (width 0.2) (layer "B.Cu") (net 30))
 (segment (start 152.8 104) (end 152.9 103.9) (width 0.2) (layer "F.Cu") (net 5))
 (segment (start 185.1 113.5) (end 185.2 113.4) (width 0.2) (layer "F.Cu") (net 11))
 (segment (start 169.88 91.4175) (end 169.88 91.56) (width 0.2) (layer "B.Cu") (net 29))
 (segment (start 164.3 85.8375) (end 169.88 91.4175) (width 0.2) (layer "B.Cu") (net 29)))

